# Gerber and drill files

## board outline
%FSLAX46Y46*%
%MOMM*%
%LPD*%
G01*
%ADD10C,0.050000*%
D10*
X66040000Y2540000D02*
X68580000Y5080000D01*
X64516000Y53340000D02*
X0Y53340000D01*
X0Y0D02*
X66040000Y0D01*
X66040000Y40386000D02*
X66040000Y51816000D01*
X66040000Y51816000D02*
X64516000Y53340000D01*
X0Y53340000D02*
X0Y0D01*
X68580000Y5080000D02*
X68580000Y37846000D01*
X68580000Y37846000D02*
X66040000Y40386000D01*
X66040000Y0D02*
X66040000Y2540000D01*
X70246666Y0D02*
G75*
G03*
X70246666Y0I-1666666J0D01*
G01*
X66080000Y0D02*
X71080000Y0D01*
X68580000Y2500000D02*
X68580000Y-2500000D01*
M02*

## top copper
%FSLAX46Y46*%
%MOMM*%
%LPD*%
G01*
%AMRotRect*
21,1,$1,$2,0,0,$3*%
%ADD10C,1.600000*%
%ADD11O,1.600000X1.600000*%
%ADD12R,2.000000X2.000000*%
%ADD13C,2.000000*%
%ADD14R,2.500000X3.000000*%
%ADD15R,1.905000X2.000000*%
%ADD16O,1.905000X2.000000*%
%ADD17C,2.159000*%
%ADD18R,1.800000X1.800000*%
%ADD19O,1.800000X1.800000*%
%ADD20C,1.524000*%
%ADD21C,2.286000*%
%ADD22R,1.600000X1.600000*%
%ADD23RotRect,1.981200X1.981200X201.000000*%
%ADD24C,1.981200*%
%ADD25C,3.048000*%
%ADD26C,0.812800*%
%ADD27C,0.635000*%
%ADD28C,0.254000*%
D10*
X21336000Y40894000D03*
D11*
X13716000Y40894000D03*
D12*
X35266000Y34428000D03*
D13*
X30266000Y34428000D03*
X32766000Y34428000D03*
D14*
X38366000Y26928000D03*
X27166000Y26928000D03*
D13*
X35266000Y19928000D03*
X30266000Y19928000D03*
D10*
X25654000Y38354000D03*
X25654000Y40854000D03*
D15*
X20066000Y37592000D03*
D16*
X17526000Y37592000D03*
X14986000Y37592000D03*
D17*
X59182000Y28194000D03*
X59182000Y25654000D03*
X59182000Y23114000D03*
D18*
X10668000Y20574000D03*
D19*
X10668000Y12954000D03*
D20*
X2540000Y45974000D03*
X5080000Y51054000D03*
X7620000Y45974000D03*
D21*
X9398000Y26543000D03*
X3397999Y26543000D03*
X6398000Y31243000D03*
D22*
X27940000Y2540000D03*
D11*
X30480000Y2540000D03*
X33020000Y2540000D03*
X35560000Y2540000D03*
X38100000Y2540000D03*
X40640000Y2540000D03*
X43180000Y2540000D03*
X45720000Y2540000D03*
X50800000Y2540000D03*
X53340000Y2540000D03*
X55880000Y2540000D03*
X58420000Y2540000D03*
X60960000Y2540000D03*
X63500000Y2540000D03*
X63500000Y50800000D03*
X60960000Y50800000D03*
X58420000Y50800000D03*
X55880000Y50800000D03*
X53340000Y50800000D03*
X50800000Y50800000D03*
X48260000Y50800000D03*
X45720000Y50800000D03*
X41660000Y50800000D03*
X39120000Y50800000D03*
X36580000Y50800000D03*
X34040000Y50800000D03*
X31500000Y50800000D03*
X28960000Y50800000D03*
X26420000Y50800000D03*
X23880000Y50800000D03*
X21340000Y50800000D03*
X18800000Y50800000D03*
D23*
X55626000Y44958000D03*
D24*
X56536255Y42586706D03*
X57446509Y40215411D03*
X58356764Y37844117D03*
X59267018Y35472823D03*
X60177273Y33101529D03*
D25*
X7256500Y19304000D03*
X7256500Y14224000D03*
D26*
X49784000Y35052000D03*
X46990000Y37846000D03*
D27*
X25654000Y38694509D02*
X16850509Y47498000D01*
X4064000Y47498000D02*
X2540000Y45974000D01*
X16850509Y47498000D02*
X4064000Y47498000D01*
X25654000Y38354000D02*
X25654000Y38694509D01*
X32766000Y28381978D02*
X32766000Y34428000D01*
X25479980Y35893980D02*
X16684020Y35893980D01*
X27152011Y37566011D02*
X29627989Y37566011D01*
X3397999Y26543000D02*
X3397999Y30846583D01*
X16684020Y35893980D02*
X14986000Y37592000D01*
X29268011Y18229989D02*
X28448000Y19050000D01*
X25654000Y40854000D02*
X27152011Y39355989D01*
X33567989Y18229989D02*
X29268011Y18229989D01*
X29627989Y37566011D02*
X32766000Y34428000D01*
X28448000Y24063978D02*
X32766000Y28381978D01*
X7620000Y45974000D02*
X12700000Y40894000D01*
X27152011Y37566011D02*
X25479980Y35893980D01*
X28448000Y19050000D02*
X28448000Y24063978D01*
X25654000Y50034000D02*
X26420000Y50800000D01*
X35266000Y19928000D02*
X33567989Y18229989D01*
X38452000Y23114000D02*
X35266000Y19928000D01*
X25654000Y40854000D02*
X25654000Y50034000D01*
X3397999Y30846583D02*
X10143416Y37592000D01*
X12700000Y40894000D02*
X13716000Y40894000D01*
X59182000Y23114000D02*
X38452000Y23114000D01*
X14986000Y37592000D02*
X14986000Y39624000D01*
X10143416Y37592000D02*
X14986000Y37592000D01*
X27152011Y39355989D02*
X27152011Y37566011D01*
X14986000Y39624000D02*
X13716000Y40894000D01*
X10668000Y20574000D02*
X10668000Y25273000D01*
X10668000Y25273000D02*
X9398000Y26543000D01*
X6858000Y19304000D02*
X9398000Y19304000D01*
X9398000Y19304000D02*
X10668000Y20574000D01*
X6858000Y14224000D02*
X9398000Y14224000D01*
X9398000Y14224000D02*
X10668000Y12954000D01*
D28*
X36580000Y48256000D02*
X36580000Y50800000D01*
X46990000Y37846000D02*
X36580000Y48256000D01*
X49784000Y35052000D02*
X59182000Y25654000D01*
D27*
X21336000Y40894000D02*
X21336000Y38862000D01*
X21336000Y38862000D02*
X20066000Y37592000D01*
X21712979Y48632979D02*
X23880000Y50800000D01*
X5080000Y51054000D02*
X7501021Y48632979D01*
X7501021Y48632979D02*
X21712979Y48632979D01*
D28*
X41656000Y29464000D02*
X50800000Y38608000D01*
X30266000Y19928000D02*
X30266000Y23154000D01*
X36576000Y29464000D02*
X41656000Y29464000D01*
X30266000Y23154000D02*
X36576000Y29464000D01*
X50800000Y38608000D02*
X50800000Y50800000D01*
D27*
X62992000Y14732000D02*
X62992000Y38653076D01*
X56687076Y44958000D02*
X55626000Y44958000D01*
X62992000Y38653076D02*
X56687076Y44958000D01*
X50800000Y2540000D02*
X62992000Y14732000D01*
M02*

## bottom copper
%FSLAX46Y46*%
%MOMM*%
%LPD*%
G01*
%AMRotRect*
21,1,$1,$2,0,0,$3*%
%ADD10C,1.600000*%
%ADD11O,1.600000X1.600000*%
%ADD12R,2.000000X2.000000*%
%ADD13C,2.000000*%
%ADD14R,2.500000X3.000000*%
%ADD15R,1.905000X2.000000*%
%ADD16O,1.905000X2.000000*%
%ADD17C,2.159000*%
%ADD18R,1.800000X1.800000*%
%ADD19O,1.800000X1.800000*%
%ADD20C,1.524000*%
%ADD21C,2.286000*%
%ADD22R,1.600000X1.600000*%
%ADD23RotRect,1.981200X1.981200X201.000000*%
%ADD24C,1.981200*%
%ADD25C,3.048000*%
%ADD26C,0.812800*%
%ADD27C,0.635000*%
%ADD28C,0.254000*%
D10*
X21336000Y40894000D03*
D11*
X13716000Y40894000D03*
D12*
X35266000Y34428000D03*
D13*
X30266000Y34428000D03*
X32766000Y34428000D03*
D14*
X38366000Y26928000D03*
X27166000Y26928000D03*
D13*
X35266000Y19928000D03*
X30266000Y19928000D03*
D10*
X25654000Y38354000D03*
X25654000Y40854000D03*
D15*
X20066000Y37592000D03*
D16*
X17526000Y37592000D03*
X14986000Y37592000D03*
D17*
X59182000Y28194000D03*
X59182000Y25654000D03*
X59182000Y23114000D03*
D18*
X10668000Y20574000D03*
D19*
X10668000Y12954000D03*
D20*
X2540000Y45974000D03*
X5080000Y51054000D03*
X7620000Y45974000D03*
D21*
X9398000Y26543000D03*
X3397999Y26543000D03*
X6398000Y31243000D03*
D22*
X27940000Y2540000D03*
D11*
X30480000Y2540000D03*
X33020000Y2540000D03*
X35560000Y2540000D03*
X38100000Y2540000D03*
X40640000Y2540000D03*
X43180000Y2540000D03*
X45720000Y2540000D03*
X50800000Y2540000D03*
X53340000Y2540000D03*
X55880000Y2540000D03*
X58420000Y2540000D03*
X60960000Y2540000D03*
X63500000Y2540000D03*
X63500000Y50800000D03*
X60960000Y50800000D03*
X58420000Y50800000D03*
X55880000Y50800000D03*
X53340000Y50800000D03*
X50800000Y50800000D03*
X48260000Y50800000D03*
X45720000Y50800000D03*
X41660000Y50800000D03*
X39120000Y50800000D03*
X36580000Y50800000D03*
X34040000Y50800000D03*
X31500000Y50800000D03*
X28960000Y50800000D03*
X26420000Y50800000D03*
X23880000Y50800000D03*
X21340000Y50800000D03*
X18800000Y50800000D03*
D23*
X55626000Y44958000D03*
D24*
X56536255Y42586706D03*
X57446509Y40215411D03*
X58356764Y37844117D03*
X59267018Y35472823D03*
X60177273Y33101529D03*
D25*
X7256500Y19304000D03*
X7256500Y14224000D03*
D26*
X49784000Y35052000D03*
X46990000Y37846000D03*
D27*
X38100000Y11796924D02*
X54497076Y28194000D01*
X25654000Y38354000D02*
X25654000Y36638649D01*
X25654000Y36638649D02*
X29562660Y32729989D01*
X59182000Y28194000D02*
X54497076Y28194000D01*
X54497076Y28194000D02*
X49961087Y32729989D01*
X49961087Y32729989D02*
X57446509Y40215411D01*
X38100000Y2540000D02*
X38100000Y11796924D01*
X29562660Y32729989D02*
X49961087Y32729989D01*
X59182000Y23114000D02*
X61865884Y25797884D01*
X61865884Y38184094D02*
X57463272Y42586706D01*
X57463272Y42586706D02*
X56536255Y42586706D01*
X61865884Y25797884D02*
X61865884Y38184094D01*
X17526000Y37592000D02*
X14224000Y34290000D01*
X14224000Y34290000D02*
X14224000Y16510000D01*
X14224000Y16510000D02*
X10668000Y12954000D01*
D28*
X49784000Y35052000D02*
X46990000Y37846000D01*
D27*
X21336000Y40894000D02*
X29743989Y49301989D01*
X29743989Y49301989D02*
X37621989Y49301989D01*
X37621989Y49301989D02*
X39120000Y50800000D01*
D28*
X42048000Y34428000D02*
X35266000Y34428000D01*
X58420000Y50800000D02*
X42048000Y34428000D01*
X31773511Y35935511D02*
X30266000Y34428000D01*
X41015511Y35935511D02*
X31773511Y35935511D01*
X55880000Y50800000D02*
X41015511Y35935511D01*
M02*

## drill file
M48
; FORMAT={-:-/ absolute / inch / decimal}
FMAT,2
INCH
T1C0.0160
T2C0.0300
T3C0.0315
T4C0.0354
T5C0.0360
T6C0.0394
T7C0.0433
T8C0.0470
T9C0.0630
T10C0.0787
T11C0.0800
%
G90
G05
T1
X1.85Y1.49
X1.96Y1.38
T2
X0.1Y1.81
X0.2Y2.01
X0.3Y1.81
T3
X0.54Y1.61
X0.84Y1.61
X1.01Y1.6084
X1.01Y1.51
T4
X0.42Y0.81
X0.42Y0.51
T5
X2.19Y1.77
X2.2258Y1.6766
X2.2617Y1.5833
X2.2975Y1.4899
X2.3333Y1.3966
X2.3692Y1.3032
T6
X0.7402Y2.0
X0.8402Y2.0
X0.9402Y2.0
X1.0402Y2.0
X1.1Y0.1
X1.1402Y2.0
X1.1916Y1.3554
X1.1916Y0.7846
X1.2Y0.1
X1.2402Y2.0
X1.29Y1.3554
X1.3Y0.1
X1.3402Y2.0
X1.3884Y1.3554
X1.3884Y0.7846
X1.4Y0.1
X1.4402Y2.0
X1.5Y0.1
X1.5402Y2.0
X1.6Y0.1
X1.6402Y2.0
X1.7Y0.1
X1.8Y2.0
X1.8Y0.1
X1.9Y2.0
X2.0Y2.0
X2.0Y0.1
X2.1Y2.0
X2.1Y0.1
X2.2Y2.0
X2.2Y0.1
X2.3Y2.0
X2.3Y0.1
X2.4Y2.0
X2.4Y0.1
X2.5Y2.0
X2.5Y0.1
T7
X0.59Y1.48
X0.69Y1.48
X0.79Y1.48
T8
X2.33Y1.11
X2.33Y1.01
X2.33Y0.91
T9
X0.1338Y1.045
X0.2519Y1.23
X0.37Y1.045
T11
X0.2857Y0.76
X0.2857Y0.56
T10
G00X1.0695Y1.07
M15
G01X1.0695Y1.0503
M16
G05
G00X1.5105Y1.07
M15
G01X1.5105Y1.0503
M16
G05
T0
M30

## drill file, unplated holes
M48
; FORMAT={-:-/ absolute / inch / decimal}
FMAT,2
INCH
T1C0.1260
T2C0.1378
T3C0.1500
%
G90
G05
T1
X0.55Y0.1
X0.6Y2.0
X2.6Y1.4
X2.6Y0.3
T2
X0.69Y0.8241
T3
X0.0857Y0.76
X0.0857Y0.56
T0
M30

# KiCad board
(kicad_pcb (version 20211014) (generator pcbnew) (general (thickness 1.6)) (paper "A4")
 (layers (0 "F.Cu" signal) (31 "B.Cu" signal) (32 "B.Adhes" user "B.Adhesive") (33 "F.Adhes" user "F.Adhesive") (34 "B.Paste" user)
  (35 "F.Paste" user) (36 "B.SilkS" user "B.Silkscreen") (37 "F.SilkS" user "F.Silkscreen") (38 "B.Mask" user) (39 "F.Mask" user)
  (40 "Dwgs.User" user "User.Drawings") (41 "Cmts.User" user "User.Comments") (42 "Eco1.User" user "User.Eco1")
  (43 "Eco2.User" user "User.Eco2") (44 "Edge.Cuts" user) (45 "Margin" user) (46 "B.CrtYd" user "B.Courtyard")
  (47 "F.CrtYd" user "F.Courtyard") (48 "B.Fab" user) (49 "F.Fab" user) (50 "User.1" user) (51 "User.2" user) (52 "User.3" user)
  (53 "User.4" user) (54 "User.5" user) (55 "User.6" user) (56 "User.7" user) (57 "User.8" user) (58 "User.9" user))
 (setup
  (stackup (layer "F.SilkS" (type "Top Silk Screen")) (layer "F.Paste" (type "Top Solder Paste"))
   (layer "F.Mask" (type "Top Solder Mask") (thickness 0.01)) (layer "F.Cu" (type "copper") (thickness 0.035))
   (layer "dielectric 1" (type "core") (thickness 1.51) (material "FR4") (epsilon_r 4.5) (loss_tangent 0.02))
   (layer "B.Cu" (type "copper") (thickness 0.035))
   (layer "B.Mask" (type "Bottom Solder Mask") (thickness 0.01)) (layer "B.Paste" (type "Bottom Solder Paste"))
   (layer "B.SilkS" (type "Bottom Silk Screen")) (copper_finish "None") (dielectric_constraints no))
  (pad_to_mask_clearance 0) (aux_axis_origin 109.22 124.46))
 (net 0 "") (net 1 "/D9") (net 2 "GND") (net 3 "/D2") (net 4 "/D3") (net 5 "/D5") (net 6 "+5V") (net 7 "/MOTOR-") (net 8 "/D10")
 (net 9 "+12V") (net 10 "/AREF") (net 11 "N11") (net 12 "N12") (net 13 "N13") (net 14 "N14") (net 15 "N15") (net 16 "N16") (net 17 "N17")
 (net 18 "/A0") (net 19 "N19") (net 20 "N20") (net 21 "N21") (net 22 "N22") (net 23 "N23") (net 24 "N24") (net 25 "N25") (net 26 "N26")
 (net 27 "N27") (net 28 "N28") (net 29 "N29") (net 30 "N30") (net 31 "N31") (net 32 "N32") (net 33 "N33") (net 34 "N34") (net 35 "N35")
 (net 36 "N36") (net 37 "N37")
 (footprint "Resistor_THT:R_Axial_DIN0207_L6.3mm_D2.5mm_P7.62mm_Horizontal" (layer "F.Cu") (at 130.556 83.566 180)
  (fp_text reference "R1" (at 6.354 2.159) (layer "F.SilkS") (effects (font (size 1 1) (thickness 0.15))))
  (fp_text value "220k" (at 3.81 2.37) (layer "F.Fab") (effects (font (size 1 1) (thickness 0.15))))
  (pad "1" thru_hole circle (at 0 0 180) (size 1.6 1.6) (drill 0.8) (layers *.Cu *.Mask) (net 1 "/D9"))
  (pad "2" thru_hole oval (at 7.62 0 180) (size 1.6 1.6) (drill 0.8) (layers *.Cu *.Mask) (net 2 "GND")))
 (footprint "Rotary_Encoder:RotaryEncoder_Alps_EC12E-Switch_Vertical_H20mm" (layer "F.Cu") (at 144.486 90.032 -90)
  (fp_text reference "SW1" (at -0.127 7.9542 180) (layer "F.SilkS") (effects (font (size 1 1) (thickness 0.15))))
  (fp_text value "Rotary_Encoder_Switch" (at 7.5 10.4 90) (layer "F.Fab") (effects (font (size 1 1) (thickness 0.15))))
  (pad "A" thru_hole rect (at 0 0 270) (size 2 2) (drill 1) (layers *.Cu *.Mask) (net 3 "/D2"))
  (pad "B" thru_hole circle (at 0 5 270) (size 2 2) (drill 1) (layers *.Cu *.Mask) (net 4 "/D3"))
  (pad "C" thru_hole circle (at 0 2.5 270) (size 2 2) (drill 1) (layers *.Cu *.Mask) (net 2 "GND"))
  (pad "MP" thru_hole rect (at 7.5 -3.1 270) (size 3 2.5) (drill oval 2.5 2) (layers *.Cu *.Mask))
  (pad "MP" thru_hole rect (at 7.5 8.1 270) (size 3 2.5) (drill oval 2.5 2) (layers *.Cu *.Mask))
  (pad "S1" thru_hole circle (at 14.5 0 270) (size 2 2) (drill 1) (layers *.Cu *.Mask) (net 2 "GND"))
  (pad "S2" thru_hole circle (at 14.5 5 270) (size 2 2) (drill 1) (layers *.Cu *.Mask) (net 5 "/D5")))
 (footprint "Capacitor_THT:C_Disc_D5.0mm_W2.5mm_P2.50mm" (layer "F.Cu") (at 134.874 86.106 90)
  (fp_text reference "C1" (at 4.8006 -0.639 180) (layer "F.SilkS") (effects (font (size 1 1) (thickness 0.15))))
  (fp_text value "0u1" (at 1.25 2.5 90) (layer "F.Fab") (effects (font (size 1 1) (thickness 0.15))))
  (pad "1" thru_hole circle (at 0 0 90) (size 1.6 1.6) (drill 0.8) (layers *.Cu *.Mask) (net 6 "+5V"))
  (pad "2" thru_hole circle (at 2.5 0 90) (size 1.6 1.6) (drill 0.8) (layers *.Cu *.Mask) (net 2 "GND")))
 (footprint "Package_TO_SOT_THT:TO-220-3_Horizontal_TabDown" (layer "F.Cu") (at 129.286 86.868 180)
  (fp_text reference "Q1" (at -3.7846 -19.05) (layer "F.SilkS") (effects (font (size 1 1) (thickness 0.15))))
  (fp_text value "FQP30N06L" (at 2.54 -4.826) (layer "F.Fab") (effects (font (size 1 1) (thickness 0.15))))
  (pad "" np_thru_hole oval (at 2.54 -16.66 180) (size 3.5 3.5) (drill 3.5) (layers *.Cu *.Mask))
  (pad "1" thru_hole rect (at 0 0 180) (size 1.905 2) (drill 1.1) (layers *.Cu *.Mask) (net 1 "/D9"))
  (pad "2" thru_hole oval (at 2.54 0 180) (size 1.905 2) (drill 1.1) (layers *.Cu *.Mask) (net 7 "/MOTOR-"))
  (pad "3" thru_hole oval (at 5.08 0 180) (size 1.905 2) (drill 1.1) (layers *.Cu *.Mask) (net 2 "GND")))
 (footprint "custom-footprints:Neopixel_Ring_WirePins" (layer "F.Cu") (at 168.402 96.266)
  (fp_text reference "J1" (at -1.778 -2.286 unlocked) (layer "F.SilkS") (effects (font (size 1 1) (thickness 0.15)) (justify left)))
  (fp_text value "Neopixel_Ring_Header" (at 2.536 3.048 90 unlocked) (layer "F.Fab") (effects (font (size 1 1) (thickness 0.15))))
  (pad "1" thru_hole circle (at 0 0) (size 2.159 2.159) (drill 1.1938) (layers *.Cu *.Mask) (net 6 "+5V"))
  (pad "2" thru_hole circle (at 0 2.54) (size 2.159 2.159) (drill 1.1938) (layers *.Cu *.Mask) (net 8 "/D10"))
  (pad "3" thru_hole circle (at 0 5.08) (size 2.159 2.159) (drill 1.1938) (layers *.Cu *.Mask) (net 2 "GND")))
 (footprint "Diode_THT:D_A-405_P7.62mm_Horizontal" (layer "F.Cu") (at 119.888 103.886 -90)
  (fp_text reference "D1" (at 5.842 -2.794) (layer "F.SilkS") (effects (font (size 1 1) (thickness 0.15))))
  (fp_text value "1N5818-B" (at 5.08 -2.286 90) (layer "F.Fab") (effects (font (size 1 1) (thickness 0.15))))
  (pad "1" thru_hole rect (at 0 0 270) (size 1.8 1.8) (drill 0.9) (layers *.Cu *.Mask) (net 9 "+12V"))
  (pad "2" thru_hole oval (at 7.62 0 270) (size 1.8 1.8) (drill 0.9) (layers *.Cu *.Mask) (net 7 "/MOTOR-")))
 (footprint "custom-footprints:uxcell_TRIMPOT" (layer "F.Cu") (at 111.76 78.486)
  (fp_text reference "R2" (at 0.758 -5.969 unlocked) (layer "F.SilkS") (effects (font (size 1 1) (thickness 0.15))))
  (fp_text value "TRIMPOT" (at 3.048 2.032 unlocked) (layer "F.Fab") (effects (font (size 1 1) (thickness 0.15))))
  (pad "1" thru_hole circle (at 0 0) (size 1.524 1.524) (drill 0.762) (layers *.Cu *.Mask) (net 6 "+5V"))
  (pad "2" thru_hole circle (at 2.54 -5.08) (size 1.524 1.524) (drill 0.762) (layers *.Cu *.Mask) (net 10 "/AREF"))
  (pad "3" thru_hole circle (at 5.08 0) (size 1.524 1.524) (drill 0.762) (layers *.Cu *.Mask) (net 2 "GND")))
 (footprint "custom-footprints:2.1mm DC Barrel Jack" (layer "B.Cu") (at 118.618 97.917 -90)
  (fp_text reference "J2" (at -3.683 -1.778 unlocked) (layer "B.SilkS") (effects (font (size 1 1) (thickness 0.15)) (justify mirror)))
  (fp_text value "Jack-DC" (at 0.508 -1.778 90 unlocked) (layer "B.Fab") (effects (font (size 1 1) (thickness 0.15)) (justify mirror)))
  (pad "1" thru_hole circle (at 0 0 270) (size 2.286 2.286) (drill 1.6002) (layers *.Cu *.Mask) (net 9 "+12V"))
  (pad "2" thru_hole circle (at 0 6.000001 270) (size 2.286 2.286) (drill 1.6002) (layers *.Cu *.Mask) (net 2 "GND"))
  (pad "3" thru_hole circle (at -4.7 3 270) (size 2.286 2.286) (drill 1.6002) (layers *.Cu *.Mask)))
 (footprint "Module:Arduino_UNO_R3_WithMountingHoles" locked (layer "B.Cu") (at 137.16 121.92)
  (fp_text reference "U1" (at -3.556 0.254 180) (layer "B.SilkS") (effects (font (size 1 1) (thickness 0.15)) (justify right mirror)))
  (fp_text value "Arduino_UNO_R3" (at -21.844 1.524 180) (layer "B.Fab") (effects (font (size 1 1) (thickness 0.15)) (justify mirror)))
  (pad "" np_thru_hole circle locked (at -12.7 -48.26 270) (size 3.2 3.2) (drill 3.2) (layers *.Cu *.Mask))
  (pad "" np_thru_hole circle locked (at 38.1 -5.08 270) (size 3.2 3.2) (drill 3.2) (layers *.Cu *.Mask))
  (pad "" np_thru_hole circle locked (at -13.97 0 270) (size 3.2 3.2) (drill 3.2) (layers *.Cu *.Mask))
  (pad "" np_thru_hole circle locked (at 38.1 -33.02 270) (size 3.2 3.2) (drill 3.2) (layers *.Cu *.Mask))
  (pad "1" thru_hole rect locked (at 0 0 270) (size 1.6 1.6) (drill 1) (layers *.Cu *.Mask) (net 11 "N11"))
  (pad "2" thru_hole oval locked (at 2.54 0 270) (size 1.6 1.6) (drill 1) (layers *.Cu *.Mask) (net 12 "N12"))
  (pad "3" thru_hole oval locked (at 5.08 0 270) (size 1.6 1.6) (drill 1) (layers *.Cu *.Mask) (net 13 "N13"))
  (pad "4" thru_hole oval locked (at 7.62 0 270) (size 1.6 1.6) (drill 1) (layers *.Cu *.Mask) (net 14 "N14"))
  (pad "5" thru_hole oval locked (at 10.16 0 270) (size 1.6 1.6) (drill 1) (layers *.Cu *.Mask) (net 6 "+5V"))
  (pad "6" thru_hole oval locked (at 12.7 0 270) (size 1.6 1.6) (drill 1) (layers *.Cu *.Mask) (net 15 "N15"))
  (pad "7" thru_hole oval locked (at 15.24 0 270) (size 1.6 1.6) (drill 1) (layers *.Cu *.Mask) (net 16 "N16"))
  (pad "8" thru_hole oval locked (at 17.78 0 270) (size 1.6 1.6) (drill 1) (layers *.Cu *.Mask) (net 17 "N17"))
  (pad "9" thru_hole oval locked (at 22.86 0 270) (size 1.6 1.6) (drill 1) (layers *.Cu *.Mask) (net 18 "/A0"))
  (pad "10" thru_hole oval locked (at 25.4 0 270) (size 1.6 1.6) (drill 1) (layers *.Cu *.Mask) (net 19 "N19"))
  (pad "11" thru_hole oval locked (at 27.94 0 270) (size 1.6 1.6) (drill 1) (layers *.Cu *.Mask) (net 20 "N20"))
  (pad "12" thru_hole oval locked (at 30.48 0 270) (size 1.6 1.6) (drill 1) (layers *.Cu *.Mask) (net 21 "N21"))
  (pad "13" thru_hole oval locked (at 33.02 0 270) (size 1.6 1.6) (drill 1) (layers *.Cu *.Mask) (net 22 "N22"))
  (pad "14" thru_hole oval locked (at 35.56 0 270) (size 1.6 1.6) (drill 1) (layers *.Cu *.Mask) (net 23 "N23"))
  (pad "15" thru_hole oval locked (at 35.56 -48.26 270) (size 1.6 1.6) (drill 1) (layers *.Cu *.Mask) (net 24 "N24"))
  (pad "16" thru_hole oval locked (at 33.02 -48.26 270) (size 1.6 1.6) (drill 1) (layers *.Cu *.Mask) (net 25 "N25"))
  (pad "17" thru_hole oval locked (at 30.48 -48.26 270) (size 1.6 1.6) (drill 1) (layers *.Cu *.Mask) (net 3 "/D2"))
  (pad "18" thru_hole oval locked (at 27.94 -48.26 270) (size 1.6 1.6) (drill 1) (layers *.Cu *.Mask) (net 4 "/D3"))
  (pad "19" thru_hole oval locked (at 25.4 -48.26 270) (size 1.6 1.6) (drill 1) (layers *.Cu *.Mask) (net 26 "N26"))
  (pad "20" thru_hole oval locked (at 22.86 -48.26 270) (size 1.6 1.6) (drill 1) (layers *.Cu *.Mask) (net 5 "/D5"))
  (pad "21" thru_hole oval locked (at 20.32 -48.26 270) (size 1.6 1.6) (drill 1) (layers *.Cu *.Mask) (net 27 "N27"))
  (pad "22" thru_hole oval locked (at 17.78 -48.26 270) (size 1.6 1.6) (drill 1) (layers *.Cu *.Mask) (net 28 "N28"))
  (pad "23" thru_hole oval locked (at 13.72 -48.26 270) (size 1.6 1.6) (drill 1) (layers *.Cu *.Mask) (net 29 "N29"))
  (pad "24" thru_hole oval locked (at 11.18 -48.26 270) (size 1.6 1.6) (drill 1) (layers *.Cu *.Mask) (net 1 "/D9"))
  (pad "25" thru_hole oval locked (at 8.64 -48.26 270) (size 1.6 1.6) (drill 1) (layers *.Cu *.Mask) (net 8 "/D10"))
  (pad "26" thru_hole oval locked (at 6.1 -48.26 270) (size 1.6 1.6) (drill 1) (layers *.Cu *.Mask) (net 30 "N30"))
  (pad "27" thru_hole oval locked (at 3.56 -48.26 270) (size 1.6 1.6) (drill 1) (layers *.Cu *.Mask) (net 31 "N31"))
  (pad "28" thru_hole oval locked (at 1.02 -48.26 270) (size 1.6 1.6) (drill 1) (layers *.Cu *.Mask) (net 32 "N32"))
  (pad "29" thru_hole oval locked (at -1.52 -48.26 270) (size 1.6 1.6) (drill 1) (layers *.Cu *.Mask) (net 2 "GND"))
  (pad "30" thru_hole oval locked (at -4.06 -48.26 270) (size 1.6 1.6) (drill 1) (layers *.Cu *.Mask) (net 10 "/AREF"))
  (pad "31" thru_hole oval locked (at -6.6 -48.26 270) (size 1.6 1.6) (drill 1) (layers *.Cu *.Mask) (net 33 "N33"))
  (pad "32" thru_hole oval locked (at -9.14 -48.26 270) (size 1.6 1.6) (drill 1) (layers *.Cu *.Mask) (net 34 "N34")))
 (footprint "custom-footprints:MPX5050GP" (layer "B.Cu") (at 164.846 79.502 -159)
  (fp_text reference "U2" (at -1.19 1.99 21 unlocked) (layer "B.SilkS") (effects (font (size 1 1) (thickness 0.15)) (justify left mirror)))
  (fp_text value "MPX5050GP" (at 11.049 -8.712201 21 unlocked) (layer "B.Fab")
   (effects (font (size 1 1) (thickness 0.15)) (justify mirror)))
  (pad "1" thru_hole rect (at 0 0 201) (size 1.9812 1.9812) (drill 0.9144) (layers *.Cu *.Mask) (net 18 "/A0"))
  (pad "2" thru_hole circle (at 0 -2.54 201) (size 1.9812 1.9812) (drill 0.9144) (layers *.Cu *.Mask) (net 2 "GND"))
  (pad "3" thru_hole circle (at 0 -5.08 201) (size 1.9812 1.9812) (drill 0.9144) (layers *.Cu *.Mask) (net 6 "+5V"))
  (pad "4" thru_hole circle (at 0 -7.62 201) (size 1.9812 1.9812) (drill 0.9144) (layers *.Cu *.Mask) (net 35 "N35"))
  (pad "5" thru_hole circle (at 0 -10.16 201) (size 1.9812 1.9812) (drill 0.9144) (layers *.Cu *.Mask) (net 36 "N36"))
  (pad "6" thru_hole circle (at 0 -12.7 201) (size 1.9812 1.9812) (drill 0.9144) (layers *.Cu *.Mask) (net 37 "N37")))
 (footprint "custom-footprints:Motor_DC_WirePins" (layer "B.Cu") (at 116.4765 105.156 180)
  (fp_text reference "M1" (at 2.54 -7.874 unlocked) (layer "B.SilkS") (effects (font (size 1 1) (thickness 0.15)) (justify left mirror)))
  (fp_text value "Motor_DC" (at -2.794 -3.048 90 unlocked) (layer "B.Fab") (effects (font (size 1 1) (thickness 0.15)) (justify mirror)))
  (pad "" np_thru_hole circle (at 5.08 0 180) (size 3.302 3.302) (drill 3.81) (layers *.Mask))
  (pad "" np_thru_hole circle (at 5.08 -5.08 180) (size 3.302 3.302) (drill 3.81) (layers *.Mask))
  (pad "1" thru_hole circle (at 0 0 180) (size 3.048 3.048) (drill 2.032) (layers *.Cu *.Mask) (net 9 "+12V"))
  (pad "2" thru_hole circle (at 0 -5.08 180) (size 3.048 3.048) (drill 2.032) (layers *.Cu *.Mask) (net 7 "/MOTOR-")))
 (gr_line (start 175.26 121.92) (end 177.8 119.38) (layer "Edge.Cuts") (width 0.05))
 (gr_line (start 173.736 71.12) (end 109.22 71.12) (layer "Edge.Cuts") (width 0.05))
 (gr_line (start 109.22 124.46) (end 175.26 124.46) (layer "Edge.Cuts") (width 0.05))
 (gr_line (start 175.26 84.074) (end 175.26 72.644) (layer "Edge.Cuts") (width 0.05))
 (gr_line (start 175.26 72.644) (end 173.736 71.12) (layer "Edge.Cuts") (width 0.05))
 (gr_line (start 109.22 71.12) (end 109.22 124.46) (layer "Edge.Cuts") (width 0.05))
 (gr_line (start 177.8 119.38) (end 177.8 86.614) (layer "Edge.Cuts") (width 0.05))
 (gr_line (start 177.8 86.614) (end 175.26 84.074) (layer "Edge.Cuts") (width 0.05))
 (gr_line (start 175.26 124.46) (end 175.26 121.92) (layer "Edge.Cuts") (width 0.05))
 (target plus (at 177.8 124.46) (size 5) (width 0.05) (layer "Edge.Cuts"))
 (segment (start 134.874 85.765491) (end 126.070509 76.962) (width 0.635) (layer "F.Cu") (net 6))
 (segment (start 113.284 76.962) (end 111.76 78.486) (width 0.635) (layer "F.Cu") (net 6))
 (segment (start 126.070509 76.962) (end 113.284 76.962) (width 0.635) (layer "F.Cu") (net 6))
 (segment (start 134.874 86.106) (end 134.874 85.765491) (width 0.635) (layer "F.Cu") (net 6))
 (segment (start 147.32 112.663076) (end 163.717076 96.266) (width 0.635) (layer "B.Cu") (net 6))
 (segment (start 134.874 86.106) (end 134.874 87.821351) (width 0.635) (layer "B.Cu") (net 6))
 (segment (start 134.874 87.821351) (end 138.78266 91.730011) (width 0.635) (layer "B.Cu") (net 6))
 (segment (start 168.402 96.266) (end 163.717076 96.266) (width 0.635) (layer "B.Cu") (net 6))
 (segment (start 163.717076 96.266) (end 159.181087 91.730011) (width 0.635) (layer "B.Cu") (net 6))
 (segment (start 159.181087 91.730011) (end 166.666509 84.244589) (width 0.635) (layer "B.Cu") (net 6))
 (segment (start 147.32 121.92) (end 147.32 112.663076) (width 0.635) (layer "B.Cu") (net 6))
 (segment (start 138.78266 91.730011) (end 159.181087 91.730011) (width 0.635) (layer "B.Cu") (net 6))
 (segment (start 141.986 96.078022) (end 141.986 90.032) (width 0.635) (layer "F.Cu") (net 2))
 (segment (start 134.69998 88.56602) (end 125.90402 88.56602) (width 0.635) (layer "F.Cu") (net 2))
 (segment (start 136.372011 86.893989) (end 138.847989 86.893989) (width 0.635) (layer "F.Cu") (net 2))
 (segment (start 112.617999 97.917) (end 112.617999 93.613417) (width 0.635) (layer "F.Cu") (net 2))
 (segment (start 125.90402 88.56602) (end 124.206 86.868) (width 0.635) (layer "F.Cu") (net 2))
 (segment (start 138.488011 106.230011) (end 137.668 105.41) (width 0.635) (layer "F.Cu") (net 2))
 (segment (start 134.874 83.606) (end 136.372011 85.104011) (width 0.635) (layer "F.Cu") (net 2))
 (segment (start 142.787989 106.230011) (end 138.488011 106.230011) (width 0.635) (layer "F.Cu") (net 2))
 (segment (start 138.847989 86.893989) (end 141.986 90.032) (width 0.635) (layer "F.Cu") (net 2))
 (segment (start 137.668 100.396022) (end 141.986 96.078022) (width 0.635) (layer "F.Cu") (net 2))
 (segment (start 116.84 78.486) (end 121.92 83.566) (width 0.635) (layer "F.Cu") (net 2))
 (segment (start 136.372011 86.893989) (end 134.69998 88.56602) (width 0.635) (layer "F.Cu") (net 2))
 (segment (start 137.668 105.41) (end 137.668 100.396022) (width 0.635) (layer "F.Cu") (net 2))
 (segment (start 134.874 74.426) (end 135.64 73.66) (width 0.635) (layer "F.Cu") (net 2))
 (segment (start 144.486 104.532) (end 142.787989 106.230011) (width 0.635) (layer "F.Cu") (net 2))
 (segment (start 147.672 101.346) (end 144.486 104.532) (width 0.635) (layer "F.Cu") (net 2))
 (segment (start 134.874 83.606) (end 134.874 74.426) (width 0.635) (layer "F.Cu") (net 2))
 (segment (start 112.617999 93.613417) (end 119.363416 86.868) (width 0.635) (layer "F.Cu") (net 2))
 (segment (start 121.92 83.566) (end 122.936 83.566) (width 0.635) (layer "F.Cu") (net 2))
 (segment (start 168.402 101.346) (end 147.672 101.346) (width 0.635) (layer "F.Cu") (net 2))
 (segment (start 124.206 86.868) (end 124.206 84.836) (width 0.635) (layer "F.Cu") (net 2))
 (segment (start 119.363416 86.868) (end 124.206 86.868) (width 0.635) (layer "F.Cu") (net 2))
 (segment (start 136.372011 85.104011) (end 136.372011 86.893989) (width 0.635) (layer "F.Cu") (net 2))
 (segment (start 124.206 84.836) (end 122.936 83.566) (width 0.635) (layer "F.Cu") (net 2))
 (segment (start 168.402 101.346) (end 171.085884 98.662116) (width 0.635) (layer "B.Cu") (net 2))
 (segment (start 171.085884 86.275906) (end 166.683272 81.873294) (width 0.635) (layer "B.Cu") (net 2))
 (segment (start 166.683272 81.873294) (end 165.756255 81.873294) (width 0.635) (layer "B.Cu") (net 2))
 (segment (start 171.085884 98.662116) (end 171.085884 86.275906) (width 0.635) (layer "B.Cu") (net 2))
 (segment (start 119.888 103.886) (end 119.888 99.187) (width 0.635) (layer "F.Cu") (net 9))
 (segment (start 119.888 99.187) (end 118.618 97.917) (width 0.635) (layer "F.Cu") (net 9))
 (segment (start 116.078 105.156) (end 118.618 105.156) (width 0.635) (layer "F.Cu") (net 9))
 (segment (start 118.618 105.156) (end 119.888 103.886) (width 0.635) (layer "F.Cu") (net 9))
 (segment (start 116.078 110.236) (end 118.618 110.236) (width 0.635) (layer "F.Cu") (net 7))
 (segment (start 118.618 110.236) (end 119.888 111.506) (width 0.635) (layer "F.Cu") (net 7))
 (segment (start 126.746 86.868) (end 123.444 90.17) (width 0.635) (layer "B.Cu") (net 7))
 (segment (start 123.444 90.17) (end 123.444 107.95) (width 0.635) (layer "B.Cu") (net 7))
 (segment (start 123.444 107.95) (end 119.888 111.506) (width 0.635) (layer "B.Cu") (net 7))
 (segment (start 145.8 76.204) (end 145.8 73.66) (width 0.254) (layer "F.Cu") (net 8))
 (segment (start 156.21 86.614) (end 145.8 76.204) (width 0.254) (layer "F.Cu") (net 8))
 (segment (start 159.004 89.408) (end 168.402 98.806) (width 0.254) (layer "F.Cu") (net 8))
 (via (at 159.004 89.408) (size 0.8128) (drill 0.4064) (layers "F.Cu" "B.Cu") (free) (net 8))
 (via (at 156.21 86.614) (size 0.8128) (drill 0.4064) (layers "F.Cu" "B.Cu") (free) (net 8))
 (segment (start 159.004 89.408) (end 156.21 86.614) (width 0.254) (layer "B.Cu") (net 8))
 (segment (start 130.556 83.566) (end 130.556 85.598) (width 0.635) (layer "F.Cu") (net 1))
 (segment (start 130.556 85.598) (end 129.286 86.868) (width 0.635) (layer "F.Cu") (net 1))
 (segment (start 130.556 83.566) (end 138.963989 75.158011) (width 0.635) (layer "B.Cu") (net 1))
 (segment (start 138.963989 75.158011) (end 146.841989 75.158011) (width 0.635) (layer "B.Cu") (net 1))
 (segment (start 146.841989 75.158011) (end 148.34 73.66) (width 0.635) (layer "B.Cu") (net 1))
 (segment (start 130.932979 75.827021) (end 133.1 73.66) (width 0.635) (layer "F.Cu") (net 10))
 (segment (start 114.3 73.406) (end 116.721021 75.827021) (width 0.635) (layer "F.Cu") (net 10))
 (segment (start 116.721021 75.827021) (end 130.932979 75.827021) (width 0.635) (layer "F.Cu") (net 10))
 (segment (start 151.268 90.032) (end 144.486 90.032) (width 0.254) (layer "B.Cu") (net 3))
 (segment (start 167.64 73.66) (end 151.268 90.032) (width 0.254) (layer "B.Cu") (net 3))
 (segment (start 140.993511 88.524489) (end 139.486 90.032) (width 0.254) (layer "B.Cu") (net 4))
 (segment (start 150.235511 88.524489) (end 140.993511 88.524489) (width 0.254) (layer "B.Cu") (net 4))
 (segment (start 165.1 73.66) (end 150.235511 88.524489) (width 0.254) (layer "B.Cu") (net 4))
 (segment (start 150.876 94.996) (end 160.02 85.852) (width 0.254) (layer "F.Cu") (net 5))
 (segment (start 139.486 104.532) (end 139.486 101.306) (width 0.254) (layer "F.Cu") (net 5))
 (segment (start 145.796 94.996) (end 150.876 94.996) (width 0.254) (layer "F.Cu") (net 5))
 (segment (start 139.486 101.306) (end 145.796 94.996) (width 0.254) (layer "F.Cu") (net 5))
 (segment (start 160.02 85.852) (end 160.02 73.66) (width 0.254) (layer "F.Cu") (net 5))
 (segment (start 172.212 109.728) (end 172.212 85.806924) (width 0.635) (layer "F.Cu") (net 18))
 (segment (start 165.907076 79.502) (end 164.846 79.502) (width 0.635) (layer "F.Cu") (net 18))
 (segment (start 172.212 85.806924) (end 165.907076 79.502) (width 0.635) (layer "F.Cu") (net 18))
 (segment (start 160.02 121.92) (end 172.212 109.728) (width 0.635) (layer "F.Cu") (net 18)))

